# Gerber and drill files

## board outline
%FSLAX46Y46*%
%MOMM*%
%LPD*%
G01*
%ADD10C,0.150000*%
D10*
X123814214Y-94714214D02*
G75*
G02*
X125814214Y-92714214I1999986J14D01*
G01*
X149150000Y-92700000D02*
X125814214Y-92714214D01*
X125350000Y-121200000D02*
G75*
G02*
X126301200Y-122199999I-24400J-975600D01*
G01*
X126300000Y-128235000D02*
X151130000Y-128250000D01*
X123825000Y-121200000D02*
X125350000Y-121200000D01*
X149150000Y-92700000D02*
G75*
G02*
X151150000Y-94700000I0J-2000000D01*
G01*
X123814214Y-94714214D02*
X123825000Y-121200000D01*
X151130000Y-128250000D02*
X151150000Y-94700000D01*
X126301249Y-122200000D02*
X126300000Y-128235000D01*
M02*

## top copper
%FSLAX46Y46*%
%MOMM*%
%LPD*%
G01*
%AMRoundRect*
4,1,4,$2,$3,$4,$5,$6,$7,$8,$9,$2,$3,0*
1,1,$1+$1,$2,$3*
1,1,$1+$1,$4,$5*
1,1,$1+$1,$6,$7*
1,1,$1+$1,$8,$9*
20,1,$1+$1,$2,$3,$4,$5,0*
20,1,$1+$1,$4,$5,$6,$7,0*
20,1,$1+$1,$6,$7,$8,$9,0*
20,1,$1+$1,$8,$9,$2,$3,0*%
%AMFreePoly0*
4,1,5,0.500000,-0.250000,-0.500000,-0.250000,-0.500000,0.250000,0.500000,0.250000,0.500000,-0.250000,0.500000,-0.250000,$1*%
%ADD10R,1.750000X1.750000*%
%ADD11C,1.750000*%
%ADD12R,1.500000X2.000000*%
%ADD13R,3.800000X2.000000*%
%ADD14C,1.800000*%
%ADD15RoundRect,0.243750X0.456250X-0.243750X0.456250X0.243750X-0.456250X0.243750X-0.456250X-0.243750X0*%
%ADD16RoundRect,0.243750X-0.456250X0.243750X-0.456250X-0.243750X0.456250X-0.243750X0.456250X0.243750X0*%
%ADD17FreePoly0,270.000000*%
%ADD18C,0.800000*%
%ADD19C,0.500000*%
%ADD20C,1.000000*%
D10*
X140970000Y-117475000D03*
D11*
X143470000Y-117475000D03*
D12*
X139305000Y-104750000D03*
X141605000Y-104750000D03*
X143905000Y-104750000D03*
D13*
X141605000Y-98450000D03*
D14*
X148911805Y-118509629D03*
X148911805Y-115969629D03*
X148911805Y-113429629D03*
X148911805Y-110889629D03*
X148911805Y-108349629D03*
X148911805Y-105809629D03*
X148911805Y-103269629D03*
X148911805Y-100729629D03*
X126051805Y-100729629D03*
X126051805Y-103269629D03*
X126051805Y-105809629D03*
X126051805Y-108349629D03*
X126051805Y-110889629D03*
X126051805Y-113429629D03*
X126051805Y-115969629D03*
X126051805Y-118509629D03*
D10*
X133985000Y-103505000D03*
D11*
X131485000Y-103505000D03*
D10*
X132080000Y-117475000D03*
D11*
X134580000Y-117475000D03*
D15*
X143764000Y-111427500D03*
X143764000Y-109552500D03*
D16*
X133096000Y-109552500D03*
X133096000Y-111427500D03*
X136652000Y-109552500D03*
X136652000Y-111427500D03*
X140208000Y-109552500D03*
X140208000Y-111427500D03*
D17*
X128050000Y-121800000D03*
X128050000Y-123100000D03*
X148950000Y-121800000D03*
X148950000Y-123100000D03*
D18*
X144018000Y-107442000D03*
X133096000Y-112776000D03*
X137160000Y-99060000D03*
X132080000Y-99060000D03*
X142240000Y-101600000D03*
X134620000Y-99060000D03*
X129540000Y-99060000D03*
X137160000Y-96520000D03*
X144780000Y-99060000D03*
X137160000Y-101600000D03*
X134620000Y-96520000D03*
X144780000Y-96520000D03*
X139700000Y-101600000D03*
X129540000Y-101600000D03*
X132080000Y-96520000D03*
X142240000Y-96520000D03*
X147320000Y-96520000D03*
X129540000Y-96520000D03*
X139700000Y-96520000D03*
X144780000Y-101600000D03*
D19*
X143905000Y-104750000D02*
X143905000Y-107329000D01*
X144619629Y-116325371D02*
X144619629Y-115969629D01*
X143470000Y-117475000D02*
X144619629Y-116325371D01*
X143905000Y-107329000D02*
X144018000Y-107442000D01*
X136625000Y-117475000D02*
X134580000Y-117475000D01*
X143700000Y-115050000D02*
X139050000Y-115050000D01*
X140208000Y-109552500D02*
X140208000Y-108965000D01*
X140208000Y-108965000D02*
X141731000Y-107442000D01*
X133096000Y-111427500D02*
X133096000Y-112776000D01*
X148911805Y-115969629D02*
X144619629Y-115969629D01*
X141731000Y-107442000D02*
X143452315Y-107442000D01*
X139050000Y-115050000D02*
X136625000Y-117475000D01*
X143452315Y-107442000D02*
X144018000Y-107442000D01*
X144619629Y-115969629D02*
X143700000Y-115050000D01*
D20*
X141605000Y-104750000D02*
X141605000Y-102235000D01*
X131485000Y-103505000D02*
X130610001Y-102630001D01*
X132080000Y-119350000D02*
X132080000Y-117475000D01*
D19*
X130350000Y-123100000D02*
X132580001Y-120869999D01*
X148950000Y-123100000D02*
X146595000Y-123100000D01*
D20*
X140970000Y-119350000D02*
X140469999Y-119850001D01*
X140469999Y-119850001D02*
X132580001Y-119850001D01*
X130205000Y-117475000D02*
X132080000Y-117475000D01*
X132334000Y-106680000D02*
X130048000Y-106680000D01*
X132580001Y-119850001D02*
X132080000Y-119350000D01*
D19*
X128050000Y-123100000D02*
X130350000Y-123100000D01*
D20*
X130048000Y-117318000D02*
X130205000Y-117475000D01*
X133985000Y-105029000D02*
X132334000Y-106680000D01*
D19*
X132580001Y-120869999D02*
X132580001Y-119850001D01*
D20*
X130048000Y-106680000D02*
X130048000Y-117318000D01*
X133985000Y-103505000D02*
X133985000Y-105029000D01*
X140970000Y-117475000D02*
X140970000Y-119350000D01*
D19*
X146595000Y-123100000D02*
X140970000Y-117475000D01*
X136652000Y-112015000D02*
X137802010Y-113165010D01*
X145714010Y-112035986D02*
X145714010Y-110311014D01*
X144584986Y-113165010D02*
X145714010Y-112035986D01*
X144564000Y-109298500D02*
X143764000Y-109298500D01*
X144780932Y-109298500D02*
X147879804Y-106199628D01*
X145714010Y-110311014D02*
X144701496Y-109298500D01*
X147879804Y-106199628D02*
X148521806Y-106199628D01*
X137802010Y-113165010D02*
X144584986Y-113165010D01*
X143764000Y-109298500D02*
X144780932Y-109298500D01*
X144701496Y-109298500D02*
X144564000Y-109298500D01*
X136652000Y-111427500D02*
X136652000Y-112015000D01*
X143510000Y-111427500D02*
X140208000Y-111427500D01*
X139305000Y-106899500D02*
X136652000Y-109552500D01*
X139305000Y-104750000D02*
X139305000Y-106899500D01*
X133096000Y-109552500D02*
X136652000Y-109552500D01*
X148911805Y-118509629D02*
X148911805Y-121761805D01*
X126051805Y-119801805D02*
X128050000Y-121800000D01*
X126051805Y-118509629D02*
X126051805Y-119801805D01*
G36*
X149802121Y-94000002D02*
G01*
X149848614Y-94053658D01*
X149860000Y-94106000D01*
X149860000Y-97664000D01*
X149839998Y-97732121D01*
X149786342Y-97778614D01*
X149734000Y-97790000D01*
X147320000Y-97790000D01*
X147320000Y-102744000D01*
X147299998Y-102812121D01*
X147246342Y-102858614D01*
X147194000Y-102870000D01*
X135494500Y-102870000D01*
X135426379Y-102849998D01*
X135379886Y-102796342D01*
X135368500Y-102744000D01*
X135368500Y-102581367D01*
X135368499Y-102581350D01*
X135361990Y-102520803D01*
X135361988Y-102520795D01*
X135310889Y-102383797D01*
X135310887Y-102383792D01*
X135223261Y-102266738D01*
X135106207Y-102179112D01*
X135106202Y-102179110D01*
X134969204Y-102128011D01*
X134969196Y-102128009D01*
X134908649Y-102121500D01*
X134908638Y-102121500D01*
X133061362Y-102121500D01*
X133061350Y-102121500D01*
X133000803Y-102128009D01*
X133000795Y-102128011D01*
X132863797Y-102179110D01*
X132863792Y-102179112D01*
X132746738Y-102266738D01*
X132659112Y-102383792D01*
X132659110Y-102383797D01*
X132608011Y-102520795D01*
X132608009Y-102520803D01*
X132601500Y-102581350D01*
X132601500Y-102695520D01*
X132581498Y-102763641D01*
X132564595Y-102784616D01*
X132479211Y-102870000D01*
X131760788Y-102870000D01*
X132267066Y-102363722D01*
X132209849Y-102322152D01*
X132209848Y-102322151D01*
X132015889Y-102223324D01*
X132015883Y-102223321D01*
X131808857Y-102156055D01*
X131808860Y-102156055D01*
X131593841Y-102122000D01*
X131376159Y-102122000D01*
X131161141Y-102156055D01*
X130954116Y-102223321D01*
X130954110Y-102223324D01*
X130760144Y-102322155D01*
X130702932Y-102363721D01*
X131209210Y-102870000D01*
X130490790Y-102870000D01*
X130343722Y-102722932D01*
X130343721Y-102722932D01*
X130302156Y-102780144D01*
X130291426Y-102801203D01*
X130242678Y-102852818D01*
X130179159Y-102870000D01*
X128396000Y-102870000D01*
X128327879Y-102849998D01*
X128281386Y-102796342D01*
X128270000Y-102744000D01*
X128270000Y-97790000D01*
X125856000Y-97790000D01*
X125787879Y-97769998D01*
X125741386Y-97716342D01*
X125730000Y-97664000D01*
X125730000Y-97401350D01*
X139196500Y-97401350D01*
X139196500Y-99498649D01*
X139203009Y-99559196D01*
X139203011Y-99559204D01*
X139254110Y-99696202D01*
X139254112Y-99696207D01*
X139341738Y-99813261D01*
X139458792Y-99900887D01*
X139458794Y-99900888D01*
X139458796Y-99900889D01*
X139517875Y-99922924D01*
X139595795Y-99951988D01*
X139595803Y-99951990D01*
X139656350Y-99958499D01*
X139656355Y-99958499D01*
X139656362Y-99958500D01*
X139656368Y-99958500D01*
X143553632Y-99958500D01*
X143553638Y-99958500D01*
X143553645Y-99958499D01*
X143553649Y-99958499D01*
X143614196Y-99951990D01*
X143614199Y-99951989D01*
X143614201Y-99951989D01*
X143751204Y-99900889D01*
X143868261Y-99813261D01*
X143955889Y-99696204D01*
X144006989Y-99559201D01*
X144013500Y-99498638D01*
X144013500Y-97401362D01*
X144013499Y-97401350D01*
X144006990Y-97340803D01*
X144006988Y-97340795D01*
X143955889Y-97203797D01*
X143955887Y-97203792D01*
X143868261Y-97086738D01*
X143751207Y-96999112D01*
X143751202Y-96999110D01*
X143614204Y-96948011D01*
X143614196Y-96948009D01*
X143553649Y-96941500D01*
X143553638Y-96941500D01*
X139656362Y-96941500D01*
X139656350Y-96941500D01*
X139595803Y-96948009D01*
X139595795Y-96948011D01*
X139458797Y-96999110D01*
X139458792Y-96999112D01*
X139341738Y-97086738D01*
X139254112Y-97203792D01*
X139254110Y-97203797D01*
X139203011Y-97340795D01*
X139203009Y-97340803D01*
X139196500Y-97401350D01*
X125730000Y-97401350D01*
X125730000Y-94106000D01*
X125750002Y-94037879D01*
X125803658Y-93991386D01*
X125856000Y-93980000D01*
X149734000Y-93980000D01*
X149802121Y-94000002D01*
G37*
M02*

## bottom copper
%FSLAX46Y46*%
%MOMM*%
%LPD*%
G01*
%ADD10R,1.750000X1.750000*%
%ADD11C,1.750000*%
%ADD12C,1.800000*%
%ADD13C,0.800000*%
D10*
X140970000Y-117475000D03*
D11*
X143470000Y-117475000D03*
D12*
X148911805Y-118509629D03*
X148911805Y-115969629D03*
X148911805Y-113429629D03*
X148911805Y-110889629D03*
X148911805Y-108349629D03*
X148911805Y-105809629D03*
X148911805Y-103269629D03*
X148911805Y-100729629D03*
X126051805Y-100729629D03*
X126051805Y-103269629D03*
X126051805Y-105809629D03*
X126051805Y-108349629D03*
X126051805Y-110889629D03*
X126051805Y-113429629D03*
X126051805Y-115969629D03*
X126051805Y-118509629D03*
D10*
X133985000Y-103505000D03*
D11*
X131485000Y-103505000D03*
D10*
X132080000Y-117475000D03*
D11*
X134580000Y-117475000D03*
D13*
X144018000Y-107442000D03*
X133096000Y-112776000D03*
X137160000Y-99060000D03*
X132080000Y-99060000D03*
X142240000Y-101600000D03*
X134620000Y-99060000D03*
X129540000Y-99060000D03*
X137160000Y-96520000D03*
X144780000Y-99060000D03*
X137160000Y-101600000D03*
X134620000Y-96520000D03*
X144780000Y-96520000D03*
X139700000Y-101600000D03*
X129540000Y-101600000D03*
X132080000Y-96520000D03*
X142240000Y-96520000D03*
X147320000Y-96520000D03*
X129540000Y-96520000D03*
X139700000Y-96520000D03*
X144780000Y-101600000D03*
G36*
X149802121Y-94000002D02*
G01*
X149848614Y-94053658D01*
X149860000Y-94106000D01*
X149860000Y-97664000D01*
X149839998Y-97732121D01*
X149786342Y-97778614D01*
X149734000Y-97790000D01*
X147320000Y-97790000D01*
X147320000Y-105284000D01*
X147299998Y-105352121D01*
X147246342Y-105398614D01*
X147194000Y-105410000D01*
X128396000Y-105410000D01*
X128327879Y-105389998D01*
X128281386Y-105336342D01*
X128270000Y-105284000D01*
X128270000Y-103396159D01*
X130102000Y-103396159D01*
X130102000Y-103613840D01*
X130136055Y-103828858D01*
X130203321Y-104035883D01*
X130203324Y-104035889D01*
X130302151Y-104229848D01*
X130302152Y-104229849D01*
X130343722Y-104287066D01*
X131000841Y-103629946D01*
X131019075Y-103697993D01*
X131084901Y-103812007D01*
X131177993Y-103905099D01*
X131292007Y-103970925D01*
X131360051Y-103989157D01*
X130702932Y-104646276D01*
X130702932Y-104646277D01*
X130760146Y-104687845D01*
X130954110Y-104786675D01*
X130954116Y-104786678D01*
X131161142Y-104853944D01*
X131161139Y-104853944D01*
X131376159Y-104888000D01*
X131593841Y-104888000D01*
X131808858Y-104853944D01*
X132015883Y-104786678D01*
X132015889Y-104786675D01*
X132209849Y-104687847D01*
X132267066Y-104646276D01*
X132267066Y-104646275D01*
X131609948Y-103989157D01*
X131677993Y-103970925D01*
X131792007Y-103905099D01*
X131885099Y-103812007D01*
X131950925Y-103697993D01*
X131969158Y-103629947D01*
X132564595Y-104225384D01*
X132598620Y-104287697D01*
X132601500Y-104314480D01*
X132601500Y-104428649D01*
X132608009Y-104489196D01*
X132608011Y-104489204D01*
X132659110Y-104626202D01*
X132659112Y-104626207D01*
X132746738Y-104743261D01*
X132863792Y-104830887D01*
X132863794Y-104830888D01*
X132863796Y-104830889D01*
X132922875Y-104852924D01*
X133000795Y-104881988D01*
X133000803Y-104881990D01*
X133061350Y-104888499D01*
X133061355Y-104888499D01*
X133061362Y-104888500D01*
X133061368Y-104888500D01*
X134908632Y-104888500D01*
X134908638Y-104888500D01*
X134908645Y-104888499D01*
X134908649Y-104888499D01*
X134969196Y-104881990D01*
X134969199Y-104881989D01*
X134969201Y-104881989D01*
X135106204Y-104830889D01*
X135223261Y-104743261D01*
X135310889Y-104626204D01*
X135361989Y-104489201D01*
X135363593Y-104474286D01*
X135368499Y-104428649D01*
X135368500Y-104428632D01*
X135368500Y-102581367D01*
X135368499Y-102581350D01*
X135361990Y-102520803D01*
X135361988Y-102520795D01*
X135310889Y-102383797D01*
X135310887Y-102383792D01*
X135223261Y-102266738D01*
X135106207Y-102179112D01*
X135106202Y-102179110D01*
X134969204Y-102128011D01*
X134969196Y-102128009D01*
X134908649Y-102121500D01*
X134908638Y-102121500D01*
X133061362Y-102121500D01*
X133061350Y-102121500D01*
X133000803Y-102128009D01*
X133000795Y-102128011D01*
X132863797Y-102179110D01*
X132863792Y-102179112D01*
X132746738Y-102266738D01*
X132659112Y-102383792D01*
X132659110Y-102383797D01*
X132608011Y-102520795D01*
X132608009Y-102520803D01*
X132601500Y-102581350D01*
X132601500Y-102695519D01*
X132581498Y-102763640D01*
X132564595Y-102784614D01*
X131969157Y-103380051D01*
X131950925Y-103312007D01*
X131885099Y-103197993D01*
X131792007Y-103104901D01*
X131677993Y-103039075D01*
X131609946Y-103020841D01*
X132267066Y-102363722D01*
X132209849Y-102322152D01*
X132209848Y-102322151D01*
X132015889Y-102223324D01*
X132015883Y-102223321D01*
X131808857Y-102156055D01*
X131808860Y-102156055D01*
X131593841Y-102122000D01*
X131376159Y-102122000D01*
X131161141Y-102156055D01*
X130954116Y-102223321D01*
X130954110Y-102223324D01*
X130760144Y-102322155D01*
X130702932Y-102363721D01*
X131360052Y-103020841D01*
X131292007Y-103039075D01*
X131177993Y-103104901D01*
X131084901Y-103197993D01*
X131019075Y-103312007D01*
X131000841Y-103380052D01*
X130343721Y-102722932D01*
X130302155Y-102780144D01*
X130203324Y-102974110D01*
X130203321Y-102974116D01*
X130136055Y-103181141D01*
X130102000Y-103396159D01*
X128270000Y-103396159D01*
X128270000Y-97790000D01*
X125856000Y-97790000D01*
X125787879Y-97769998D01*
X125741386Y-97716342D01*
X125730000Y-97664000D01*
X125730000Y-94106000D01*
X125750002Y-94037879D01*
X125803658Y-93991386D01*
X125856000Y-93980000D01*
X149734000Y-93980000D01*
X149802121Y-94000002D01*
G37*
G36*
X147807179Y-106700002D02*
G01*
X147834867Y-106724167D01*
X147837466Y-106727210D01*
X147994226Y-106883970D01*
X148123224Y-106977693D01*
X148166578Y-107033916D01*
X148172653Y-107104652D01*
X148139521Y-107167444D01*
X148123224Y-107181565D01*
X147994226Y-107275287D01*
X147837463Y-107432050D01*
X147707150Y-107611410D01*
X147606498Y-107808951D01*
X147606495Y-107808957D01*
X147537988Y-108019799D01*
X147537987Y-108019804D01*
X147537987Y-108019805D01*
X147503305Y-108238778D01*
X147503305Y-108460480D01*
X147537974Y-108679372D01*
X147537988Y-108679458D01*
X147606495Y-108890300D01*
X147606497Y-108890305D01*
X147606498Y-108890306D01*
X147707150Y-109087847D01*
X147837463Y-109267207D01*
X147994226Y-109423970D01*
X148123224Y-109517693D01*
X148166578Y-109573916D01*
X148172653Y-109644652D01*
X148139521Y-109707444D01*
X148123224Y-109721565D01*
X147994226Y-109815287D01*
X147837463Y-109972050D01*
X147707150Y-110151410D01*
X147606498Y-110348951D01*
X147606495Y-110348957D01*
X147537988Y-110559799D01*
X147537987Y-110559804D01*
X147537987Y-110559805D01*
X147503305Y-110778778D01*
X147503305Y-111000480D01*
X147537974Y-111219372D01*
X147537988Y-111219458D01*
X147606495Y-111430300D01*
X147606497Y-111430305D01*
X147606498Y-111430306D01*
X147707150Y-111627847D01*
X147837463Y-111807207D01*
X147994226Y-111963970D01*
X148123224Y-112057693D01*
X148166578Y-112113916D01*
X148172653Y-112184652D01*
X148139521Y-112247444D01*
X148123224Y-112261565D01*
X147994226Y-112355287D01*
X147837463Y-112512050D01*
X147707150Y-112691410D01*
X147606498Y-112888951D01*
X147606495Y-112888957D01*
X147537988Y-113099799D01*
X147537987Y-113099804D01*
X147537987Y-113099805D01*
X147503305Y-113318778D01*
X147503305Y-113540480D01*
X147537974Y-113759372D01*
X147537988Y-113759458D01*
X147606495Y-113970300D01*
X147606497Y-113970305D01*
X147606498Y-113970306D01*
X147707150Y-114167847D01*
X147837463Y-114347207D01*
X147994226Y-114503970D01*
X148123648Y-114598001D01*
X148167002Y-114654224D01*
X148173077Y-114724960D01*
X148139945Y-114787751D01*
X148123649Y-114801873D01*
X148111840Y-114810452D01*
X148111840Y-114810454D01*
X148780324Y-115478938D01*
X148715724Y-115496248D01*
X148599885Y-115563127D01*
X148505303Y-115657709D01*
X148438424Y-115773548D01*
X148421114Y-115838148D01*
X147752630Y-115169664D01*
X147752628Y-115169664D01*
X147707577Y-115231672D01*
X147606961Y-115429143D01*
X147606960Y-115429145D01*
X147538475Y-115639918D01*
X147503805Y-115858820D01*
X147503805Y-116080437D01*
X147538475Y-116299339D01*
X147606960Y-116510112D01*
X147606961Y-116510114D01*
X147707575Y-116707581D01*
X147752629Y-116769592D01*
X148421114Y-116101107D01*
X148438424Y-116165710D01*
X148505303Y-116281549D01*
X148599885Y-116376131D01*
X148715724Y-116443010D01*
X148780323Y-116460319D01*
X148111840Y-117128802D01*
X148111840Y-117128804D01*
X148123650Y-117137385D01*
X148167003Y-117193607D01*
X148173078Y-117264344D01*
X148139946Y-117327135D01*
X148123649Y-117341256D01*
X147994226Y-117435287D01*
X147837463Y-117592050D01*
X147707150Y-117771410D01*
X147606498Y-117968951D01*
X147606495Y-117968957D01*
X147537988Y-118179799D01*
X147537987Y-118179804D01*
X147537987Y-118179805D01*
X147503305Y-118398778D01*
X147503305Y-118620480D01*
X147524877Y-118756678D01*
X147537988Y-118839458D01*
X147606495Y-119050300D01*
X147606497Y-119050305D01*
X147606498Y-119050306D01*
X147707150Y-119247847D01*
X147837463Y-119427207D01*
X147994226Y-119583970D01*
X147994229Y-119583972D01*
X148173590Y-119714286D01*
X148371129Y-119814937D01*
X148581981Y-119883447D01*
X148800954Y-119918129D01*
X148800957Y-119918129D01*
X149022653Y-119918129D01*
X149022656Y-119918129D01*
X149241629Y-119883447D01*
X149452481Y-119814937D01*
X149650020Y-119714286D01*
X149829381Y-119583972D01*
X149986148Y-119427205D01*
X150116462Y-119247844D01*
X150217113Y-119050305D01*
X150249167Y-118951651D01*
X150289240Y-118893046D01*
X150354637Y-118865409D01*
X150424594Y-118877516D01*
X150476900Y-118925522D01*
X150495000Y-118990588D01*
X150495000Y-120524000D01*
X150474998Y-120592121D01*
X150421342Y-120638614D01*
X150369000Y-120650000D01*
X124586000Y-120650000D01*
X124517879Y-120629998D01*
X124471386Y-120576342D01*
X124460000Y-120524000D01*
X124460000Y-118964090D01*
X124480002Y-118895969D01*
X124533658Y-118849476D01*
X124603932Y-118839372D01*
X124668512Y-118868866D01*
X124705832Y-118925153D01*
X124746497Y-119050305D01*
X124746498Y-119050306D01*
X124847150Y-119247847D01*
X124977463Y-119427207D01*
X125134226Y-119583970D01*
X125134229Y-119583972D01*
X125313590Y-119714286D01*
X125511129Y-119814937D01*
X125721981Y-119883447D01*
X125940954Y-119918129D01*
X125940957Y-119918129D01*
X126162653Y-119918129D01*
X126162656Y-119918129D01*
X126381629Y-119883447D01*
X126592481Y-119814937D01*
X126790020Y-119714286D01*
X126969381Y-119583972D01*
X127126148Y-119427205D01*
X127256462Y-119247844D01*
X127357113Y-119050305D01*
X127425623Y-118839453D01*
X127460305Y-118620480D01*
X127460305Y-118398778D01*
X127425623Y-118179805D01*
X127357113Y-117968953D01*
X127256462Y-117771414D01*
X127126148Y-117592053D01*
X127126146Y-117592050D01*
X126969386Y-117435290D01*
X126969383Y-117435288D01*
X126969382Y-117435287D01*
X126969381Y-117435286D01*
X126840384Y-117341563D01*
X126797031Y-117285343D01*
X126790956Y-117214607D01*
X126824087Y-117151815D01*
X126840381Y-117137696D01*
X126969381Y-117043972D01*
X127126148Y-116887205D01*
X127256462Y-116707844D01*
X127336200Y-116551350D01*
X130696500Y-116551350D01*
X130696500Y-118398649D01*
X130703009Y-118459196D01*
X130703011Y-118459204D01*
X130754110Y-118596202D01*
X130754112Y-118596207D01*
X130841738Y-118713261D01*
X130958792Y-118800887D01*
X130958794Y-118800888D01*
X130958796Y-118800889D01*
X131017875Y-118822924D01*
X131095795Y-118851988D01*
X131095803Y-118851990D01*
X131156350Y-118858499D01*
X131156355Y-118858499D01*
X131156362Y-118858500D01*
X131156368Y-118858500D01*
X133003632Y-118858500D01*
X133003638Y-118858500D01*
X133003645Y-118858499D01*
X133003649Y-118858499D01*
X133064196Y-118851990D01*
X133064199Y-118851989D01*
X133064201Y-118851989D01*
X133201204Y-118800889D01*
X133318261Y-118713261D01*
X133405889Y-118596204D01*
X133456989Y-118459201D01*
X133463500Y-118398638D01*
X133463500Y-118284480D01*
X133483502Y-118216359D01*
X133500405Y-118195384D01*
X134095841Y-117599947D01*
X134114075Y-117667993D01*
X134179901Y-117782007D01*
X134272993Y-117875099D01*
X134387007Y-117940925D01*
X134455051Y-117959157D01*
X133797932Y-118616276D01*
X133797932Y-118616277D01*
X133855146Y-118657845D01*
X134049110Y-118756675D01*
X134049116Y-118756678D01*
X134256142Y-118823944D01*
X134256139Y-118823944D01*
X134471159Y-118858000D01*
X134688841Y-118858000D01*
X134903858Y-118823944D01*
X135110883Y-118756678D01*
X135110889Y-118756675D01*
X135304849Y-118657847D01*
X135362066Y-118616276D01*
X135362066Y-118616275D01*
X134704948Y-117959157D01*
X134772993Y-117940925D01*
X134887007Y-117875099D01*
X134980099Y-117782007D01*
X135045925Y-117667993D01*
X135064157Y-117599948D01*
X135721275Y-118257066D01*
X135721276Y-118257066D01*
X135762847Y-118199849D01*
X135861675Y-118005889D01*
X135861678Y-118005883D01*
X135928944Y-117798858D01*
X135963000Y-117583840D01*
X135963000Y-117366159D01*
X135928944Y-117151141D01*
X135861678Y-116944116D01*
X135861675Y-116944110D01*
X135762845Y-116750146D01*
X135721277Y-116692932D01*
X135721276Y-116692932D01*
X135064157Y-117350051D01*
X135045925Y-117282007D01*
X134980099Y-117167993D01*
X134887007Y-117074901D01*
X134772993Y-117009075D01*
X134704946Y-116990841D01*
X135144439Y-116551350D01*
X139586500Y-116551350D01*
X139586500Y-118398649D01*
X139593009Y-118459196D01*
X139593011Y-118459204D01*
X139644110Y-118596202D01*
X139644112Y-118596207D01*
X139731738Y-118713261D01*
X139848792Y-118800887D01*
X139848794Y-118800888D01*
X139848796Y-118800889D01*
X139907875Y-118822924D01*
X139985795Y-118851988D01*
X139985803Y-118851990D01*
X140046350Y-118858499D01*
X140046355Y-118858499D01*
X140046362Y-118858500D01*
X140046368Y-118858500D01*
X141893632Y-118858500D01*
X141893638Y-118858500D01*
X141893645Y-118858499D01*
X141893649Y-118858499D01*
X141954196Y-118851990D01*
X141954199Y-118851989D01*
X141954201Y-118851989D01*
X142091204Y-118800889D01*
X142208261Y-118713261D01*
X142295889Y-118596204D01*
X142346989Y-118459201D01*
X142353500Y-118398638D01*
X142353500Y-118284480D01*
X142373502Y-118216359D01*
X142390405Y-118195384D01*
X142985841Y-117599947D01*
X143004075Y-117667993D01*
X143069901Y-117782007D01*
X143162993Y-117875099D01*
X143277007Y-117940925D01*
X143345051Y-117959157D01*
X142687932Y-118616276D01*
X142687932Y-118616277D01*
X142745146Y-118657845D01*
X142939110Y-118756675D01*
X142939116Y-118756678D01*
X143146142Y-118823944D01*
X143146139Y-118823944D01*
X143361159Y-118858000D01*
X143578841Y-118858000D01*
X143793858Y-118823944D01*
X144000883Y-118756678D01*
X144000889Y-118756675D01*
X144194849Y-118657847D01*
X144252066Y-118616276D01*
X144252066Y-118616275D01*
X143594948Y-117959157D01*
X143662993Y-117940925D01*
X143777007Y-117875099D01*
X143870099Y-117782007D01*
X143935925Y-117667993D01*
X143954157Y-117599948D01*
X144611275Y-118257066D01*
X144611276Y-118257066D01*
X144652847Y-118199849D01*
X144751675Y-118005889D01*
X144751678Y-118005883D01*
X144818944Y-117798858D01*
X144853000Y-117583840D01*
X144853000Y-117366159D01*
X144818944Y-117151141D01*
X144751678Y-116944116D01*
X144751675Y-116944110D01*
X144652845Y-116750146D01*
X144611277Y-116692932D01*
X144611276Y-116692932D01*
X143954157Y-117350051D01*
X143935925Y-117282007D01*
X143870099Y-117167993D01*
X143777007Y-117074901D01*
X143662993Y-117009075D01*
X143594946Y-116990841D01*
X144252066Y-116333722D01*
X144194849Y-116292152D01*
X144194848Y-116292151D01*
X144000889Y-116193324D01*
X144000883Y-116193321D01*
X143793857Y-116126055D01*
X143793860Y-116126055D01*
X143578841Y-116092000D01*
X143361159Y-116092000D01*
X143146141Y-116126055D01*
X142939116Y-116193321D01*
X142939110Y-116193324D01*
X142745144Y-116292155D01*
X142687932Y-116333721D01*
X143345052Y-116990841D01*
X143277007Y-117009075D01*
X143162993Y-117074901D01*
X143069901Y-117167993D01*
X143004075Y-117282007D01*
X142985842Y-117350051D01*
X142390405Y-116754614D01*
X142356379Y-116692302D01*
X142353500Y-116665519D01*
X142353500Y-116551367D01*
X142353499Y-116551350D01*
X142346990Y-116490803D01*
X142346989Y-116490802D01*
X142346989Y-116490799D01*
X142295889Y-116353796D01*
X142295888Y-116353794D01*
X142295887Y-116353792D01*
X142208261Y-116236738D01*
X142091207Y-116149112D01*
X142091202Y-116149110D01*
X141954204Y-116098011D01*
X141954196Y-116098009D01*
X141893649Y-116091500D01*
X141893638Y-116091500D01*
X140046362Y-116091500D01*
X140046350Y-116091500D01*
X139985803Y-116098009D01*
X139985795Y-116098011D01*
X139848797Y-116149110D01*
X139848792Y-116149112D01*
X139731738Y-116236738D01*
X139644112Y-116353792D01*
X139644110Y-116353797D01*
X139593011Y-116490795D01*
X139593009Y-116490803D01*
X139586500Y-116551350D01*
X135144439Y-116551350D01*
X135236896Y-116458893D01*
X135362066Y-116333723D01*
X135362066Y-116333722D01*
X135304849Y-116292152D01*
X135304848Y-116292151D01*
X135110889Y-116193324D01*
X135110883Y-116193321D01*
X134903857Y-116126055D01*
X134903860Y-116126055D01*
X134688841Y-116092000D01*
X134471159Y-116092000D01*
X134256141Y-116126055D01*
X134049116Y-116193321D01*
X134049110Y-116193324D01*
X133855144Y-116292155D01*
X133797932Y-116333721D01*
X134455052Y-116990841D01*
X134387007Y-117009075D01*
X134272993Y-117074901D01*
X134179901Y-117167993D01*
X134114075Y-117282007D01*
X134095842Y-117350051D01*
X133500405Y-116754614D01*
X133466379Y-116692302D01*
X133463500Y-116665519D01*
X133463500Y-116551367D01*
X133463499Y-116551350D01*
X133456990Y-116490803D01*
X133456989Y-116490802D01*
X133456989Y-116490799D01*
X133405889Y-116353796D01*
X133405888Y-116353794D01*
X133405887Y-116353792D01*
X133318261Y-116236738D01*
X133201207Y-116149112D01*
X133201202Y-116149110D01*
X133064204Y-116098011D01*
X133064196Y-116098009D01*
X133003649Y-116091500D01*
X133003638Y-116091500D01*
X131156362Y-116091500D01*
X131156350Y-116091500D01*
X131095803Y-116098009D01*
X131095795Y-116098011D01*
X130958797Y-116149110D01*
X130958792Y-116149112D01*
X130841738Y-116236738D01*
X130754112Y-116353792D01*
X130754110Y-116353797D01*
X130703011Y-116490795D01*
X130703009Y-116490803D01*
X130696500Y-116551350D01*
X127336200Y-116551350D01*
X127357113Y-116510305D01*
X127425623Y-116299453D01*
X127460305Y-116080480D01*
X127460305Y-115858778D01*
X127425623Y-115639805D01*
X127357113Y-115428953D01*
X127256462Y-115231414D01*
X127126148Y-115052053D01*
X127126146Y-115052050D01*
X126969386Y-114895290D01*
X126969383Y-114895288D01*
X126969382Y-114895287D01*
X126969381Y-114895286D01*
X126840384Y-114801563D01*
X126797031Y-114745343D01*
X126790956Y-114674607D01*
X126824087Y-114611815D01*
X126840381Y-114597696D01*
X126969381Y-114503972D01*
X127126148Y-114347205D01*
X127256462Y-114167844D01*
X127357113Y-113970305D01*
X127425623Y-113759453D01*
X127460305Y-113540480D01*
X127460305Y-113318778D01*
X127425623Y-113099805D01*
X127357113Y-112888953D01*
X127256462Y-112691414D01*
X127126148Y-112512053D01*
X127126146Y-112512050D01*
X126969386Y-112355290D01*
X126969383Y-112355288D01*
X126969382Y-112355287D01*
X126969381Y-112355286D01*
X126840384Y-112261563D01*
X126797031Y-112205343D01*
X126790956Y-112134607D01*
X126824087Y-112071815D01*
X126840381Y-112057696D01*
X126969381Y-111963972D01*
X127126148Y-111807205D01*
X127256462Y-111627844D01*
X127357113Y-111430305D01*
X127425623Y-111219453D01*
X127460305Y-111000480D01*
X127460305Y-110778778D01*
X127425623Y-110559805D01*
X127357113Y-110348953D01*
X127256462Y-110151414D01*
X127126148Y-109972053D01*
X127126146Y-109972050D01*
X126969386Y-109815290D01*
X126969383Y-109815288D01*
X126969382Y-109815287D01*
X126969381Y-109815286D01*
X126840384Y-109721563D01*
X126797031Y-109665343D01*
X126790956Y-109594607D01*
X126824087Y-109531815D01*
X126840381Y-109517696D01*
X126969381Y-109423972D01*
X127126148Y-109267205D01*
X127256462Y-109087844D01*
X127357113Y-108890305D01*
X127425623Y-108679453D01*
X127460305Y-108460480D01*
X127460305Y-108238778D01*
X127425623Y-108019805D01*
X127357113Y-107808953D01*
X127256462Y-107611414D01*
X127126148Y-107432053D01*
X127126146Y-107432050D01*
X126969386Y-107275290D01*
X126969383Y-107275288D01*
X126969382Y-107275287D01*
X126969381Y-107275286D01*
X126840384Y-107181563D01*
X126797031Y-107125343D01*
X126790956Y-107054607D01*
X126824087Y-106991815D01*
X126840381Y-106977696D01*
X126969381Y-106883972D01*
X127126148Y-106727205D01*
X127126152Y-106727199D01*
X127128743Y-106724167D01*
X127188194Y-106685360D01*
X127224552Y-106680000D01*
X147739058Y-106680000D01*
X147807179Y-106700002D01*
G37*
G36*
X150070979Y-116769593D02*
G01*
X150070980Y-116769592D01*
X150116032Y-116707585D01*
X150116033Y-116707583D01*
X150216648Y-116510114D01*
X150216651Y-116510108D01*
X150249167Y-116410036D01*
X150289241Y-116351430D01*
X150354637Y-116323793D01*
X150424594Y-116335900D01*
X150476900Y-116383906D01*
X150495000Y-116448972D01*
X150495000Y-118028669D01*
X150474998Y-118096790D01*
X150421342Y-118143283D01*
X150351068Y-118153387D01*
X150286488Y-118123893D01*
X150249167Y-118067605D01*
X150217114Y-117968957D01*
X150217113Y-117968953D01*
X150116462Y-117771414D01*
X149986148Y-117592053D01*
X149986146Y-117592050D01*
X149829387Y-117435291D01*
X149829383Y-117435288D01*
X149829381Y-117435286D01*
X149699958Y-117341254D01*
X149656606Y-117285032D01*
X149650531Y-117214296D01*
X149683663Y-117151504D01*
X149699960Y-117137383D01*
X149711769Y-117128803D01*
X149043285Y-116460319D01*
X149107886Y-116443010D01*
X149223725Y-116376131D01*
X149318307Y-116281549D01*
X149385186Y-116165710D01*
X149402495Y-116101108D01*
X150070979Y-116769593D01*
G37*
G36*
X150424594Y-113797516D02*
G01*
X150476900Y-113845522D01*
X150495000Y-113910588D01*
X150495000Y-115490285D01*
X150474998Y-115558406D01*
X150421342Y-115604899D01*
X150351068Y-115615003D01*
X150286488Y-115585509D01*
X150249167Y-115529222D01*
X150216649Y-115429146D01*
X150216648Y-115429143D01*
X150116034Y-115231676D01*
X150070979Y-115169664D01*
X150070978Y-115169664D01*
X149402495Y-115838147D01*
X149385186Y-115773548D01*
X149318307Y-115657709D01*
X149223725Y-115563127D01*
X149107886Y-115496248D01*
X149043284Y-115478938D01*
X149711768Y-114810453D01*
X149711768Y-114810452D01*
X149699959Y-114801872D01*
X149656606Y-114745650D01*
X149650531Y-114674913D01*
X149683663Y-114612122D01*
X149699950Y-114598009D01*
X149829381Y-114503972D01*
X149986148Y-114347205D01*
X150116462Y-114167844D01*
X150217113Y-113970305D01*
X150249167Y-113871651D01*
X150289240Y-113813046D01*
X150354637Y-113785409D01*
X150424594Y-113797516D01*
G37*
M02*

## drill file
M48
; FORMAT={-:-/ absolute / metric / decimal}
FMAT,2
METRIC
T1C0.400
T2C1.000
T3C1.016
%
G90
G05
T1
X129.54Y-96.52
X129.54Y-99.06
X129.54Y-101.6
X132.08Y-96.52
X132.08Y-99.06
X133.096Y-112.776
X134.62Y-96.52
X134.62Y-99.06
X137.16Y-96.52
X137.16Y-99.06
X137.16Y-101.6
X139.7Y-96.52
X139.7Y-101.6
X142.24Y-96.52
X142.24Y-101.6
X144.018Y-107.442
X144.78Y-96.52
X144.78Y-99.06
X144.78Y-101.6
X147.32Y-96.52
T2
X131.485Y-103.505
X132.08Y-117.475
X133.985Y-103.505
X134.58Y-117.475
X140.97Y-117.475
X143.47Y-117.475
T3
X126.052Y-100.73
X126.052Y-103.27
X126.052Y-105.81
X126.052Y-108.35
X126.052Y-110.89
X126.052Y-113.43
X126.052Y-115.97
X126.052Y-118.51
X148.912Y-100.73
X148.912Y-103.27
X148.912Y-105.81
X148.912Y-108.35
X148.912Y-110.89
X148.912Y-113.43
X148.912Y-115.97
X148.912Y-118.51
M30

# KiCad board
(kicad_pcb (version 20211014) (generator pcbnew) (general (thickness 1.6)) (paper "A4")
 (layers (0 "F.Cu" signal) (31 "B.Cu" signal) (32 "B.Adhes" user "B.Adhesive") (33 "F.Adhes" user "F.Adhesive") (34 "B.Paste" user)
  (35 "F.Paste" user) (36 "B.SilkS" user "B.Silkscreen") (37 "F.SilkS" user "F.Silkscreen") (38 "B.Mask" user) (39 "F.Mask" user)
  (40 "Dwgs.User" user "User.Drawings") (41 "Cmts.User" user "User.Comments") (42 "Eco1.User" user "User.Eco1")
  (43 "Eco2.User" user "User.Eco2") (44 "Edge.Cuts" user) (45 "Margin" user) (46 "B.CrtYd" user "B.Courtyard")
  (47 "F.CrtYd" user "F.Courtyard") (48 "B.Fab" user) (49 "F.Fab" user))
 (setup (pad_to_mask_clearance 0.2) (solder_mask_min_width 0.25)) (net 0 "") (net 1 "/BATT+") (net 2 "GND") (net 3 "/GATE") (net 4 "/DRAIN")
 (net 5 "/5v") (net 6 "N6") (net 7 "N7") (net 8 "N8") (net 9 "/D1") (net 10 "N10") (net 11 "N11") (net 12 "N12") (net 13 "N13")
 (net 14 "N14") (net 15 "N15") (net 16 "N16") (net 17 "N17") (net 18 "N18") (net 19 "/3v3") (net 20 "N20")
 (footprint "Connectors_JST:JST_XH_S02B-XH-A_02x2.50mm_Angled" (layer "F.Cu") (at 140.97 117.475)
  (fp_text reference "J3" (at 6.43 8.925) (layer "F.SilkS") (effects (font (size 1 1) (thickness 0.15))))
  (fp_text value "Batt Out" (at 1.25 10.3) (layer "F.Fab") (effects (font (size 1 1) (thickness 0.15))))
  (pad "1" thru_hole rect locked (at 0 0) (size 1.75 1.75) (drill 1) (layers *.Cu *.Mask) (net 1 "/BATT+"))
  (pad "2" thru_hole circle locked (at 2.5 0) (size 1.75 1.75) (drill 1) (layers *.Cu *.Mask) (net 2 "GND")))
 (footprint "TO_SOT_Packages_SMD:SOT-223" (layer "F.Cu") (at 141.605 101.6 90)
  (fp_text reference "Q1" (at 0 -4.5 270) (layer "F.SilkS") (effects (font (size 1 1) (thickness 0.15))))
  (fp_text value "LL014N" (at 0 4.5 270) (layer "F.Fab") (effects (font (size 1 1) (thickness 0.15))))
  (pad "1" smd rect locked (at -3.15 -2.3 90) (size 2 1.5) (layers "F.Cu" "F.Paste" "F.Mask") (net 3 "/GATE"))
  (pad "2" smd rect locked (at -3.15 0 90) (size 2 1.5) (layers "F.Cu" "F.Paste" "F.Mask") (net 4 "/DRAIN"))
  (pad "3" smd rect locked (at -3.15 2.3 90) (size 2 1.5) (layers "F.Cu" "F.Paste" "F.Mask") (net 2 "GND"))
  (pad "4" smd rect locked (at 3.15 0 90) (size 2 3.8) (layers "F.Cu" "F.Paste" "F.Mask")))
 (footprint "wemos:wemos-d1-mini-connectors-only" (layer "F.Cu") (at 137.481805 109.619629 90)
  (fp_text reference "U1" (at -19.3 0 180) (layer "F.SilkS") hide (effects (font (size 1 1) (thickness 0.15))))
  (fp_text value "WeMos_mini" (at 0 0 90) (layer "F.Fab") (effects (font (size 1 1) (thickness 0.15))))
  (pad "1" thru_hole circle locked (at -8.89 11.43 90) (size 1.8 1.8) (drill 1.016) (layers *.Cu *.Mask) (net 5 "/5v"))
  (pad "2" thru_hole circle locked (at -6.35 11.43 90) (size 1.8 1.8) (drill 1.016) (layers *.Cu *.Mask) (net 2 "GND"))
  (pad "3" thru_hole circle locked (at -3.81 11.43 90) (size 1.8 1.8) (drill 1.016) (layers *.Cu *.Mask) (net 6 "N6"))
  (pad "4" thru_hole circle locked (at -1.27 11.43 90) (size 1.8 1.8) (drill 1.016) (layers *.Cu *.Mask) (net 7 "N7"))
  (pad "5" thru_hole circle locked (at 1.27 11.43 90) (size 1.8 1.8) (drill 1.016) (layers *.Cu *.Mask) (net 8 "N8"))
  (pad "6" thru_hole circle locked (at 3.81 11.43 90) (size 1.8 1.8) (drill 1.016) (layers *.Cu *.Mask) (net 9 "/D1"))
  (pad "7" thru_hole circle locked (at 6.35 11.43 90) (size 1.8 1.8) (drill 1.016) (layers *.Cu *.Mask) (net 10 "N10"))
  (pad "8" thru_hole circle locked (at 8.89 11.43 90) (size 1.8 1.8) (drill 1.016) (layers *.Cu *.Mask) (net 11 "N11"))
  (pad "9" thru_hole circle locked (at 8.89 -11.43 90) (size 1.8 1.8) (drill 1.016) (layers *.Cu *.Mask) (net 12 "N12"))
  (pad "10" thru_hole circle locked (at 6.35 -11.43 90) (size 1.8 1.8) (drill 1.016) (layers *.Cu *.Mask) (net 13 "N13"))
  (pad "11" thru_hole circle locked (at 3.81 -11.43 90) (size 1.8 1.8) (drill 1.016) (layers *.Cu *.Mask) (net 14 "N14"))
  (pad "12" thru_hole circle locked (at 1.27 -11.43 90) (size 1.8 1.8) (drill 1.016) (layers *.Cu *.Mask) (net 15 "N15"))
  (pad "13" thru_hole circle locked (at -1.27 -11.43 90) (size 1.8 1.8) (drill 1.016) (layers *.Cu *.Mask) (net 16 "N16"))
  (pad "14" thru_hole circle locked (at -3.81 -11.43 90) (size 1.8 1.8) (drill 1.016) (layers *.Cu *.Mask) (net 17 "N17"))
  (pad "15" thru_hole circle locked (at -6.35 -11.43 90) (size 1.8 1.8) (drill 1.016) (layers *.Cu *.Mask) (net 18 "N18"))
  (pad "16" thru_hole circle locked (at -8.89 -11.43 90) (size 1.8 1.8) (drill 1.016) (layers *.Cu *.Mask) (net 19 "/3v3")))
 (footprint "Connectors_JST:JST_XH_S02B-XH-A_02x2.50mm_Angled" (layer "F.Cu") (at 133.985 103.505 180)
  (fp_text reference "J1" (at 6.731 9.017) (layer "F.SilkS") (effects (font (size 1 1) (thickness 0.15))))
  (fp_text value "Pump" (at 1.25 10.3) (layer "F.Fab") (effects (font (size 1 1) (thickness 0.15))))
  (pad "1" thru_hole rect locked (at 0 0 180) (size 1.75 1.75) (drill 1) (layers *.Cu *.Mask) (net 1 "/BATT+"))
  (pad "2" thru_hole circle locked (at 2.5 0 180) (size 1.75 1.75) (drill 1) (layers *.Cu *.Mask) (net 4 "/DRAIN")))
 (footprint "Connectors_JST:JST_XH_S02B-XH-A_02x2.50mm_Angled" (layer "F.Cu") (at 132.08 117.475)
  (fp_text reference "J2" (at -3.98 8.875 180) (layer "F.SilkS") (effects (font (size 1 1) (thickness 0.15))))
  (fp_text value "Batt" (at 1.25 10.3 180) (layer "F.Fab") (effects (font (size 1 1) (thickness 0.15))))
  (pad "1" thru_hole rect locked (at 0 0) (size 1.75 1.75) (drill 1) (layers *.Cu *.Mask) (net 1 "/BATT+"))
  (pad "2" thru_hole circle locked (at 2.5 0) (size 1.75 1.75) (drill 1) (layers *.Cu *.Mask) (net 2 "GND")))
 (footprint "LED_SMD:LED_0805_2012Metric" (layer "F.Cu") (at 143.764 110.49 90)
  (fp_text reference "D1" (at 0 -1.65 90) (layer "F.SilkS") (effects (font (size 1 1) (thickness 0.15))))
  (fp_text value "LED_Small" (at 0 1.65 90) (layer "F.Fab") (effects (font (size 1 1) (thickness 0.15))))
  (pad "1" smd roundrect locked (at -0.9375 0 90) (size 0.975 1.4) (layers "F.Cu" "F.Paste" "F.Mask") (roundrect_rratio 0.25) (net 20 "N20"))
  (pad "2" smd roundrect locked (at 0.9375 0 90) (size 0.975 1.4) (layers "F.Cu" "F.Paste" "F.Mask") (roundrect_rratio 0.25) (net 9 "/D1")))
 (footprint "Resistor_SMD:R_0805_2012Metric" (layer "F.Cu") (at 133.096 110.49 -90)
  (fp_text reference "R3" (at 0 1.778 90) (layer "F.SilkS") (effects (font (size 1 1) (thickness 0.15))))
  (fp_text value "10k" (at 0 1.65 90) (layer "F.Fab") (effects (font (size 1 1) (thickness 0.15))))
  (pad "1" smd roundrect locked (at -0.9375 0 270) (size 0.975 1.4) (layers "F.Cu" "F.Paste" "F.Mask") (roundrect_rratio 0.25)
   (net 3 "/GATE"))
  (pad "2" smd roundrect locked (at 0.9375 0 270) (size 0.975 1.4) (layers "F.Cu" "F.Paste" "F.Mask") (roundrect_rratio 0.25) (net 2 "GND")))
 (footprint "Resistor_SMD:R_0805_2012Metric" (layer "F.Cu") (at 136.652 110.49 -90)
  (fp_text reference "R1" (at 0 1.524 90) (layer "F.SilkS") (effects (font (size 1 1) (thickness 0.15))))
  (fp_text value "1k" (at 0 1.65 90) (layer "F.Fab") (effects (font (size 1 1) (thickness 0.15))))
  (pad "1" smd roundrect locked (at -0.9375 0 270) (size 0.975 1.4) (layers "F.Cu" "F.Paste" "F.Mask") (roundrect_rratio 0.25)
   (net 3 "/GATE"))
  (pad "2" smd roundrect locked (at 0.9375 0 270) (size 0.975 1.4) (layers "F.Cu" "F.Paste" "F.Mask") (roundrect_rratio 0.25) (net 9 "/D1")))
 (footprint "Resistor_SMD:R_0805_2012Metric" (layer "F.Cu") (at 140.208 110.49 -90)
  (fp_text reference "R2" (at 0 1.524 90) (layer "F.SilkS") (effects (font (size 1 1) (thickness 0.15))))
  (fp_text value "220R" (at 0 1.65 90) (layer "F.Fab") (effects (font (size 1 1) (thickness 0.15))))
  (pad "1" smd roundrect locked (at -0.9375 0 270) (size 0.975 1.4) (layers "F.Cu" "F.Paste" "F.Mask") (roundrect_rratio 0.25) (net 2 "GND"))
  (pad "2" smd roundrect locked (at 0.9375 0 270) (size 0.975 1.4) (layers "F.Cu" "F.Paste" "F.Mask") (roundrect_rratio 0.25) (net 20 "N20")))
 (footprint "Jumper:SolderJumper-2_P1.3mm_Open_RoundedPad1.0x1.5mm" (layer "F.Cu") (at 128.05 122.45 -90)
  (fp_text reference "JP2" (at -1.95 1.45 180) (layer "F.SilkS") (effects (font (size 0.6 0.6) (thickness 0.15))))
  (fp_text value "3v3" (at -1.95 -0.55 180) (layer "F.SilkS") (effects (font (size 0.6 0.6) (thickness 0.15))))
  (pad "1" smd custom (at -0.65 0 270) (size 1 0.5) (layers "F.Cu" "F.Mask") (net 19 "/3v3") (zone_connect 2)
   (options (clearance outline) (anchor rect)) (primitives))
  (pad "2" smd custom (at 0.65 0 270) (size 1 0.5) (layers "F.Cu" "F.Mask") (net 1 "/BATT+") (zone_connect 2)
   (options (clearance outline) (anchor rect)) (primitives)))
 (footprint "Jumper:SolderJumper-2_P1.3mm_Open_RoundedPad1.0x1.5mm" (layer "F.Cu") (at 148.95 122.45 -90)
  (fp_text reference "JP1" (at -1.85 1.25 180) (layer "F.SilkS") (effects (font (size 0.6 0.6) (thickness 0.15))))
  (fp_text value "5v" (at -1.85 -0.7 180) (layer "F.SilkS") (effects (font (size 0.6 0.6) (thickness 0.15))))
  (pad "1" smd custom (at -0.65 0 270) (size 1 0.5) (layers "F.Cu" "F.Mask") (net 5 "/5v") (zone_connect 2)
   (options (clearance outline) (anchor rect)) (primitives))
  (pad "2" smd custom (at 0.65 0 270) (size 1 0.5) (layers "F.Cu" "F.Mask") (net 1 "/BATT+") (zone_connect 2)
   (options (clearance outline) (anchor rect)) (primitives)))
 (gr_arc (start 123.814214 94.714214) (mid 124.4 93.3) (end 125.814214 92.714214) (layer "Edge.Cuts") (width 0.15))
 (gr_line (start 149.15 92.7) (end 125.814214 92.714214) (layer "Edge.Cuts") (width 0.15))
 (gr_arc (start 125.35 121.2) (mid 126.032732 121.50299) (end 126.301249 122.2) (layer "Edge.Cuts") (width 0.15))
 (gr_line (start 126.3 128.235) (end 151.13 128.25) (layer "Edge.Cuts") (width 0.15))
 (gr_line (start 123.825 121.2) (end 125.35 121.2) (layer "Edge.Cuts") (width 0.15))
 (gr_arc (start 149.15 92.7) (mid 150.564214 93.285786) (end 151.15 94.7) (layer "Edge.Cuts") (width 0.15))
 (gr_line (start 123.814214 94.714214) (end 123.825 121.2) (layer "Edge.Cuts") (width 0.15))
 (gr_line (start 151.13 128.25) (end 151.15 94.7) (layer "Edge.Cuts") (width 0.15))
 (gr_line (start 126.301249 122.2) (end 126.3 128.235) (layer "Edge.Cuts") (width 0.15))
 (segment (start 143.905 104.75) (end 143.905 107.329) (width 0.5) (layer "F.Cu") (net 2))
 (segment (start 144.619629 116.325371) (end 144.619629 115.969629) (width 0.5) (layer "F.Cu") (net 2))
 (segment (start 143.47 117.475) (end 144.619629 116.325371) (width 0.5) (layer "F.Cu") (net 2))
 (segment (start 143.905 107.329) (end 144.018 107.442) (width 0.5) (layer "F.Cu") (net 2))
 (segment (start 136.625 117.475) (end 134.58 117.475) (width 0.5) (layer "F.Cu") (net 2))
 (segment (start 143.7 115.05) (end 139.05 115.05) (width 0.5) (layer "F.Cu") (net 2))
 (segment (start 140.208 109.5525) (end 140.208 108.965) (width 0.5) (layer "F.Cu") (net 2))
 (segment (start 140.208 108.965) (end 141.731 107.442) (width 0.5) (layer "F.Cu") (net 2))
 (segment (start 133.096 111.4275) (end 133.096 112.776) (width 0.5) (layer "F.Cu") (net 2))
 (segment (start 148.911805 115.969629) (end 144.619629 115.969629) (width 0.5) (layer "F.Cu") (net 2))
 (segment (start 141.731 107.442) (end 143.452315 107.442) (width 0.5) (layer "F.Cu") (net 2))
 (segment (start 139.05 115.05) (end 136.625 117.475) (width 0.5) (layer "F.Cu") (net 2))
 (segment (start 143.452315 107.442) (end 144.018 107.442) (width 0.5) (layer "F.Cu") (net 2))
 (segment (start 144.619629 115.969629) (end 143.7 115.05) (width 0.5) (layer "F.Cu") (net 2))
 (via (at 144.018 107.442) (size 0.8) (drill 0.4) (layers "F.Cu" "B.Cu") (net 2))
 (via (at 133.096 112.776) (size 0.8) (drill 0.4) (layers "F.Cu" "B.Cu") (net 2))
 (segment (start 141.605 104.75) (end 141.605 102.235) (width 1) (layer "F.Cu") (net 4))
 (segment (start 131.485 103.505) (end 130.610001 102.630001) (width 1) (layer "F.Cu") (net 4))
 (via (at 137.16 99.06) (size 0.8) (drill 0.4) (layers "F.Cu" "B.Cu") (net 4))
 (via (at 132.08 99.06) (size 0.8) (drill 0.4) (layers "F.Cu" "B.Cu") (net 4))
 (via (at 142.24 101.6) (size 0.8) (drill 0.4) (layers "F.Cu" "B.Cu") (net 4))
 (via (at 134.62 99.06) (size 0.8) (drill 0.4) (layers "F.Cu" "B.Cu") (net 4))
 (via (at 129.54 99.06) (size 0.8) (drill 0.4) (layers "F.Cu" "B.Cu") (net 4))
 (via (at 137.16 96.52) (size 0.8) (drill 0.4) (layers "F.Cu" "B.Cu") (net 4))
 (via (at 144.78 99.06) (size 0.8) (drill 0.4) (layers "F.Cu" "B.Cu") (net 4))
 (via (at 137.16 101.6) (size 0.8) (drill 0.4) (layers "F.Cu" "B.Cu") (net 4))
 (via (at 134.62 96.52) (size 0.8) (drill 0.4) (layers "F.Cu" "B.Cu") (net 4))
 (via (at 144.78 96.52) (size 0.8) (drill 0.4) (layers "F.Cu" "B.Cu") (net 4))
 (via (at 139.7 101.6) (size 0.8) (drill 0.4) (layers "F.Cu" "B.Cu") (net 4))
 (via (at 129.54 101.6) (size 0.8) (drill 0.4) (layers "F.Cu" "B.Cu") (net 4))
 (via (at 132.08 96.52) (size 0.8) (drill 0.4) (layers "F.Cu" "B.Cu") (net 4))
 (via (at 142.24 96.52) (size 0.8) (drill 0.4) (layers "F.Cu" "B.Cu") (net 4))
 (via (at 147.32 96.52) (size 0.8) (drill 0.4) (layers "F.Cu" "B.Cu") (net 4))
 (via (at 129.54 96.52) (size 0.8) (drill 0.4) (layers "F.Cu" "B.Cu") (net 4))
 (via (at 139.7 96.52) (size 0.8) (drill 0.4) (layers "F.Cu" "B.Cu") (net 4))
 (via (at 144.78 101.6) (size 0.8) (drill 0.4) (layers "F.Cu" "B.Cu") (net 4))
 (segment (start 132.08 119.35) (end 132.08 117.475) (width 1) (layer "F.Cu") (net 1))
 (segment (start 130.35 123.1) (end 132.580001 120.869999) (width 0.5) (layer "F.Cu") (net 1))
 (segment (start 148.95 123.1) (end 146.595 123.1) (width 0.5) (layer "F.Cu") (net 1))
 (segment (start 140.97 119.35) (end 140.469999 119.850001) (width 1) (layer "F.Cu") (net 1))
 (segment (start 140.469999 119.850001) (end 132.580001 119.850001) (width 1) (layer "F.Cu") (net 1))
 (segment (start 130.205 117.475) (end 132.08 117.475) (width 1) (layer "F.Cu") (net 1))
 (segment (start 132.334 106.68) (end 130.048 106.68) (width 1) (layer "F.Cu") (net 1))
 (segment (start 132.580001 119.850001) (end 132.08 119.35) (width 1) (layer "F.Cu") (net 1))
 (segment (start 128.05 123.1) (end 130.35 123.1) (width 0.5) (layer "F.Cu") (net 1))
 (segment (start 130.048 117.318) (end 130.205 117.475) (width 1) (layer "F.Cu") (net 1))
 (segment (start 133.985 105.029) (end 132.334 106.68) (width 1) (layer "F.Cu") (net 1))
 (segment (start 132.580001 120.869999) (end 132.580001 119.850001) (width 0.5) (layer "F.Cu") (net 1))
 (segment (start 130.048 106.68) (end 130.048 117.318) (width 1) (layer "F.Cu") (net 1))
 (segment (start 133.985 103.505) (end 133.985 105.029) (width 1) (layer "F.Cu") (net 1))
 (segment (start 140.97 117.475) (end 140.97 119.35) (width 1) (layer "F.Cu") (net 1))
 (segment (start 146.595 123.1) (end 140.97 117.475) (width 0.5) (layer "F.Cu") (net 1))
 (segment (start 136.652 112.015) (end 137.80201 113.16501) (width 0.5) (layer "F.Cu") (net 9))
 (segment (start 145.71401 112.035986) (end 145.71401 110.311014) (width 0.5) (layer "F.Cu") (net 9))
 (segment (start 144.584986 113.16501) (end 145.71401 112.035986) (width 0.5) (layer "F.Cu") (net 9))
 (segment (start 144.564 109.2985) (end 143.764 109.2985) (width 0.5) (layer "F.Cu") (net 9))
 (segment (start 144.780932 109.2985) (end 147.879804 106.199628) (width 0.5) (layer "F.Cu") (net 9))
 (segment (start 145.71401 110.311014) (end 144.701496 109.2985) (width 0.5) (layer "F.Cu") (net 9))
 (segment (start 147.879804 106.199628) (end 148.521806 106.199628) (width 0.5) (layer "F.Cu") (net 9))
 (segment (start 137.80201 113.16501) (end 144.584986 113.16501) (width 0.5) (layer "F.Cu") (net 9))
 (segment (start 143.764 109.2985) (end 144.780932 109.2985) (width 0.5) (layer "F.Cu") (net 9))
 (segment (start 144.701496 109.2985) (end 144.564 109.2985) (width 0.5) (layer "F.Cu") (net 9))
 (segment (start 136.652 111.4275) (end 136.652 112.015) (width 0.5) (layer "F.Cu") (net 9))
 (segment (start 143.51 111.4275) (end 140.208 111.4275) (width 0.5) (layer "F.Cu") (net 20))
 (segment (start 139.305 106.8995) (end 136.652 109.5525) (width 0.5) (layer "F.Cu") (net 3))
 (segment (start 139.305 104.75) (end 139.305 106.8995) (width 0.5) (layer "F.Cu") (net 3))
 (segment (start 133.096 109.5525) (end 136.652 109.5525) (width 0.5) (layer "F.Cu") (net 3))
 (segment (start 148.911805 118.509629) (end 148.911805 121.761805) (width 0.5) (layer "F.Cu") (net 5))
 (segment (start 126.051805 119.801805) (end 128.05 121.8) (width 0.5) (layer "F.Cu") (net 19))
 (segment (start 126.051805 118.509629) (end 126.051805 119.801805) (width 0.5) (layer "F.Cu") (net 19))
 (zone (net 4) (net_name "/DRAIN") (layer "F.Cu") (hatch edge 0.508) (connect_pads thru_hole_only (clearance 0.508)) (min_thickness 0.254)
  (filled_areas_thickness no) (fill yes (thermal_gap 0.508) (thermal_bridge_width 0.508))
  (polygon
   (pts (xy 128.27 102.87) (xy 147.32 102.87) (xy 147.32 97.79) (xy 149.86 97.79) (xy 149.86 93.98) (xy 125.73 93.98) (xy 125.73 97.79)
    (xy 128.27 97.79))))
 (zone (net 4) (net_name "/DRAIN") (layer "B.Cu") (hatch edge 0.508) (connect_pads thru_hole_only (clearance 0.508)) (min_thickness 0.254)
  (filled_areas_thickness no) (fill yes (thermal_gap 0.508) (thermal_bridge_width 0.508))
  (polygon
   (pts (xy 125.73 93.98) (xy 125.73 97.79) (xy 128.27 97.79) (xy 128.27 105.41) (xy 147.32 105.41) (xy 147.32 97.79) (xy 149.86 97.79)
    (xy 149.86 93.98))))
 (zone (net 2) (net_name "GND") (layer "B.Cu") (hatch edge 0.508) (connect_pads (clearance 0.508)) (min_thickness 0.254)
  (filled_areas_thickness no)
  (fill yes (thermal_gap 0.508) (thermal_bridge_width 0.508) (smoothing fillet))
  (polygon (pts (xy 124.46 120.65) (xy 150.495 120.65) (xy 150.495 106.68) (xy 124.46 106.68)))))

